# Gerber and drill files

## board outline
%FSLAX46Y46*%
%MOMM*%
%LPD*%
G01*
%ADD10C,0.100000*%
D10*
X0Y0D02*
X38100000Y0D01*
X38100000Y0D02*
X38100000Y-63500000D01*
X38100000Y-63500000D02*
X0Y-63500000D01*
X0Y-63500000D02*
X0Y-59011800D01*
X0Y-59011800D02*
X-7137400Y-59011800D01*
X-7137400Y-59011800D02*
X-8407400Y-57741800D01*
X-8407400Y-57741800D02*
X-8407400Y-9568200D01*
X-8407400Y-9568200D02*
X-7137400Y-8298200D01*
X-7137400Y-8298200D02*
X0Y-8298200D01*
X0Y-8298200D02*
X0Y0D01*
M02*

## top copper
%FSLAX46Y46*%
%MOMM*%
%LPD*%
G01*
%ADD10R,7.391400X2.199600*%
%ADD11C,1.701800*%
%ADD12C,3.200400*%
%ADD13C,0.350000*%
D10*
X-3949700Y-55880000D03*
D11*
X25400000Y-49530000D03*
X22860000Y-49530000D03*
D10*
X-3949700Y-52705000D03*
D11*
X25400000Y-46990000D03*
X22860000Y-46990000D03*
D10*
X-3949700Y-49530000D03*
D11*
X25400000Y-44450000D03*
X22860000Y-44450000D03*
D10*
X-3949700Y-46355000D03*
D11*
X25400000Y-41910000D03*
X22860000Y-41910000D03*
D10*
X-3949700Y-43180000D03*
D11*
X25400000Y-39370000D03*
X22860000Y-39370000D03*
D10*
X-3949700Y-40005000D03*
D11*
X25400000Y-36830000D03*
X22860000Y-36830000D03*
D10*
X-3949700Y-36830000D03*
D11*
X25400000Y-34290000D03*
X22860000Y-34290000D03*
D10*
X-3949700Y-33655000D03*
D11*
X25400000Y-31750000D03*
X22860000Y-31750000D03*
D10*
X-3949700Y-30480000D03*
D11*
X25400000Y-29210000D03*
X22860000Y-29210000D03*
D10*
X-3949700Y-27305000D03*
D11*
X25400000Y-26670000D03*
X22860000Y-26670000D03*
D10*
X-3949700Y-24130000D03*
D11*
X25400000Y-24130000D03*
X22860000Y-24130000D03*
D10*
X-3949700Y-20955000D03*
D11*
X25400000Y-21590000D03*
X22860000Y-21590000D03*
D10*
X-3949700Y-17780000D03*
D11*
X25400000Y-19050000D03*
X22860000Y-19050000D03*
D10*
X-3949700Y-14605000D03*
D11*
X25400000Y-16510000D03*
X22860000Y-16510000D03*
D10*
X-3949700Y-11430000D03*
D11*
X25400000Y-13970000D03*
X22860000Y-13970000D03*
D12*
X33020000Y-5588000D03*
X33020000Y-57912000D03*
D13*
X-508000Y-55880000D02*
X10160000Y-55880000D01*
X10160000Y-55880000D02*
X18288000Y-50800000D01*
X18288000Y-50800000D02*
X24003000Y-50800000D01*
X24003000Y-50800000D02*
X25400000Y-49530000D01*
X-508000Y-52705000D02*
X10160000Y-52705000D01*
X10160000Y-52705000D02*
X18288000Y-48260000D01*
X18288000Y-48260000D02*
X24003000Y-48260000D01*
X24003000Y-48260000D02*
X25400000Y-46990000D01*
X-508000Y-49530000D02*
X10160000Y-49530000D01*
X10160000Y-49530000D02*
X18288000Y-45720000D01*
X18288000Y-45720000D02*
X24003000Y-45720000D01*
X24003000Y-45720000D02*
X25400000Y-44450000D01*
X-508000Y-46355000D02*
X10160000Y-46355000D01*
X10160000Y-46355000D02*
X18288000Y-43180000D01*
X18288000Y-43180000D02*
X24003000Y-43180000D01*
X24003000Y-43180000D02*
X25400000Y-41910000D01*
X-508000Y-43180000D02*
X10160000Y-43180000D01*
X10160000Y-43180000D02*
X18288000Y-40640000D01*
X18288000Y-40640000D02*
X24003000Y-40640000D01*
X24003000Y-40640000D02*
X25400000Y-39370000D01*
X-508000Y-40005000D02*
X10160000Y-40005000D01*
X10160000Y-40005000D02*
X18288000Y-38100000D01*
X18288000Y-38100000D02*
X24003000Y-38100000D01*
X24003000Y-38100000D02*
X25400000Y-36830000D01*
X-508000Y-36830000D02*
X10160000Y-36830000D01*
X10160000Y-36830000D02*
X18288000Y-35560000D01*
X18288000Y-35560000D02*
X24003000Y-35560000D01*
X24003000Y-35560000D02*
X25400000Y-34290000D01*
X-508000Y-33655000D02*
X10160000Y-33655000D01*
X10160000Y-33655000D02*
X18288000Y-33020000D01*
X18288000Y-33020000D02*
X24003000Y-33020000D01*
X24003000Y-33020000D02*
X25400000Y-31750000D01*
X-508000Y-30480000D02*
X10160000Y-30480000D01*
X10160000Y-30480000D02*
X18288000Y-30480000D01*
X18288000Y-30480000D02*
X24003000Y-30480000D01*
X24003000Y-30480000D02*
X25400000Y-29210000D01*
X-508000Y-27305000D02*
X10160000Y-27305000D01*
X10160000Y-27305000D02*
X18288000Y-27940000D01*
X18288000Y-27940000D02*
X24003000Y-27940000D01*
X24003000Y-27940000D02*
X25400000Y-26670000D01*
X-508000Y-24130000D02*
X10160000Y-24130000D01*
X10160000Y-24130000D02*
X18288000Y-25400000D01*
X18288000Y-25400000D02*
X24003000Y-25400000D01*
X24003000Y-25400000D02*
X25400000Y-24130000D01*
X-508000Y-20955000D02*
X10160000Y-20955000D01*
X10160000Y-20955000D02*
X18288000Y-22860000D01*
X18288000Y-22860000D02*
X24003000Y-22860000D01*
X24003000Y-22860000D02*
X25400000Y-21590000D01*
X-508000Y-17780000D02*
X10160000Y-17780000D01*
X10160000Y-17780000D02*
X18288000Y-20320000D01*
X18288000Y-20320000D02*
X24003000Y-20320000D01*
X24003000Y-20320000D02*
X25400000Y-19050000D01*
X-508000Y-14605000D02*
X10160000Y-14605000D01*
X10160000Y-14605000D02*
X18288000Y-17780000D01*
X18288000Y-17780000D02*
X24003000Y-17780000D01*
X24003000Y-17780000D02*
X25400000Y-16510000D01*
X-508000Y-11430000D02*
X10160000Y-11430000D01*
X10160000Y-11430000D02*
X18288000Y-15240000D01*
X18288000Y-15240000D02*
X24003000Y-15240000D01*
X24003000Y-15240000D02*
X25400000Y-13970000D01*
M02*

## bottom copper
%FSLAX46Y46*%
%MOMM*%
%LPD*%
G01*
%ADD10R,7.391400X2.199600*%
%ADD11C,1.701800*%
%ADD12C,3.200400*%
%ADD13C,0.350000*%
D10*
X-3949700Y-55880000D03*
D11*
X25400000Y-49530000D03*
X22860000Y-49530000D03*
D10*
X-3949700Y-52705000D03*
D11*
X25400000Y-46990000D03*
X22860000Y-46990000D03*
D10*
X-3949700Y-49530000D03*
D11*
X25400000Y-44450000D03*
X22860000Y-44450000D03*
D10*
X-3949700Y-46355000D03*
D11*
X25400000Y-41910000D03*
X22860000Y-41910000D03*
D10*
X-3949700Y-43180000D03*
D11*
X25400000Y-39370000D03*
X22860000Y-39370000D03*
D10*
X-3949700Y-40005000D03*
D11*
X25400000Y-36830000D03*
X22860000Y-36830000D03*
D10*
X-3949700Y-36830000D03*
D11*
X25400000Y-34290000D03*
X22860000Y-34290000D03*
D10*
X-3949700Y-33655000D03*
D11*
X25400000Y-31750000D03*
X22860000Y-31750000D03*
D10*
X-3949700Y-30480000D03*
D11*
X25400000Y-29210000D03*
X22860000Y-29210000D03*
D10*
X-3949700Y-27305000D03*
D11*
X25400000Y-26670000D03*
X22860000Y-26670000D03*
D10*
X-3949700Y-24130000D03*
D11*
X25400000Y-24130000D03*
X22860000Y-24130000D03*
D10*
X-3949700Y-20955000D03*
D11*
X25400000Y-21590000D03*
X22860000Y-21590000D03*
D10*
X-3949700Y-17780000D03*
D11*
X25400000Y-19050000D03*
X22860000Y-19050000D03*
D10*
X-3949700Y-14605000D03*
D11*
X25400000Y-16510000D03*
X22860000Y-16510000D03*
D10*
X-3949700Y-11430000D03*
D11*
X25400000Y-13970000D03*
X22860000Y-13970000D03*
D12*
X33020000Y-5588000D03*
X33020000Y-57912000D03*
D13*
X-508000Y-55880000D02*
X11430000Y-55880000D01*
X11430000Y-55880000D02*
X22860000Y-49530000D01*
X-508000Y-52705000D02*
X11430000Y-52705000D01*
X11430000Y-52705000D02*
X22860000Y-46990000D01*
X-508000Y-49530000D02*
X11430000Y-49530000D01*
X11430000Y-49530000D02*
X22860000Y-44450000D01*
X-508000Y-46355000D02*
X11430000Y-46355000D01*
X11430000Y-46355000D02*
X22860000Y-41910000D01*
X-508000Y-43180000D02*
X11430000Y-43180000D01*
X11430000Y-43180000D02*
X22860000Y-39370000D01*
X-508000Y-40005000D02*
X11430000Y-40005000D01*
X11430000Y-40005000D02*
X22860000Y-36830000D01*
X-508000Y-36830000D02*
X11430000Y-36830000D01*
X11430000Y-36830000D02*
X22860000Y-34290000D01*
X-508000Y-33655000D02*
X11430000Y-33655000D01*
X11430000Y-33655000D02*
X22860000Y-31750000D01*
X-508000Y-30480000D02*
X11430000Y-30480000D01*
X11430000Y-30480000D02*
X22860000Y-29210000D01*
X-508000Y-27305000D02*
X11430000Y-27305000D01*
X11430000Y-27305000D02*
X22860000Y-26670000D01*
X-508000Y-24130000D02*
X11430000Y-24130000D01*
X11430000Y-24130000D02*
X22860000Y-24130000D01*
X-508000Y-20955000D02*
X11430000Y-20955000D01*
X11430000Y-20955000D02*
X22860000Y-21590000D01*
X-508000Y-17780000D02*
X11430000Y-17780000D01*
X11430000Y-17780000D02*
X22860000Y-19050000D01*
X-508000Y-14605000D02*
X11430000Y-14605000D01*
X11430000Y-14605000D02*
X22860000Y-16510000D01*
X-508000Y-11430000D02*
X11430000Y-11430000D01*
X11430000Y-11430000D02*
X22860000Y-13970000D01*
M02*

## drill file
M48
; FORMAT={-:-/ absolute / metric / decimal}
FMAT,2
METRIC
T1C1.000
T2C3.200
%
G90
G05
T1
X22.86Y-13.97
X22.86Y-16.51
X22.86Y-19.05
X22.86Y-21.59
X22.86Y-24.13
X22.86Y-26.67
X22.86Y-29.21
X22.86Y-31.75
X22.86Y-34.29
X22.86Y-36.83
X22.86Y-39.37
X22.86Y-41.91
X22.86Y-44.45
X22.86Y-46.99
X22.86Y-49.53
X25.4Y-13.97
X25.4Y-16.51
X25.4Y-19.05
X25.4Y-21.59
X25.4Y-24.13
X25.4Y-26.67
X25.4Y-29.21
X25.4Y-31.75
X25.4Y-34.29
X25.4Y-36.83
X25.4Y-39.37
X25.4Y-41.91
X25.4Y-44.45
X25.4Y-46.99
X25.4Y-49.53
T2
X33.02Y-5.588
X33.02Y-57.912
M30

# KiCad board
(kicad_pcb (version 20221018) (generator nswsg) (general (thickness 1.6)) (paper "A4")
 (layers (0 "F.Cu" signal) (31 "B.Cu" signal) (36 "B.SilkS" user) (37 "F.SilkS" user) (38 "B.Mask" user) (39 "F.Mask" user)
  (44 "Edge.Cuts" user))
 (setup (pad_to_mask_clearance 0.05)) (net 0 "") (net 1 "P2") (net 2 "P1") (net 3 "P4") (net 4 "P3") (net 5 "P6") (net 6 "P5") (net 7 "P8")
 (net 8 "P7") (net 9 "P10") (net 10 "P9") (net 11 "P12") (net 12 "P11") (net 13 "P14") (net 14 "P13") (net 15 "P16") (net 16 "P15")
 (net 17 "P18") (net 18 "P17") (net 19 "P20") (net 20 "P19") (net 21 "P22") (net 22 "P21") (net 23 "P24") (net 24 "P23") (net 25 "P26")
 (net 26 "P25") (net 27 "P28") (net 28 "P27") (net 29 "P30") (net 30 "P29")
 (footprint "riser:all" (layer "F.Cu") (at 0 0)
  (pad "2" smd rect (at -3.9497 55.88) (size 7.3914 2.1996) (layers "F.Cu" "F.Mask") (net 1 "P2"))
  (pad "1" smd rect (at -3.9497 55.88) (size 7.3914 2.1996) (layers "B.Cu" "B.Mask") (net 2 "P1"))
  (pad "2" thru_hole circle (at 25.4 49.53) (size 1.7018 1.7018) (drill 1.0) (layers "*.Cu" "*.Mask") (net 1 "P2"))
  (pad "1" thru_hole circle (at 22.86 49.53) (size 1.7018 1.7018) (drill 1.0) (layers "*.Cu" "*.Mask") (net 2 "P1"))
  (pad "4" smd rect (at -3.9497 52.705) (size 7.3914 2.1996) (layers "F.Cu" "F.Mask") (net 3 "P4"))
  (pad "3" smd rect (at -3.9497 52.705) (size 7.3914 2.1996) (layers "B.Cu" "B.Mask") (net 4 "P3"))
  (pad "4" thru_hole circle (at 25.4 46.99) (size 1.7018 1.7018) (drill 1.0) (layers "*.Cu" "*.Mask") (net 3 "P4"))
  (pad "3" thru_hole circle (at 22.86 46.99) (size 1.7018 1.7018) (drill 1.0) (layers "*.Cu" "*.Mask") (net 4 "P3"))
  (pad "6" smd rect (at -3.9497 49.53) (size 7.3914 2.1996) (layers "F.Cu" "F.Mask") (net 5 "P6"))
  (pad "5" smd rect (at -3.9497 49.53) (size 7.3914 2.1996) (layers "B.Cu" "B.Mask") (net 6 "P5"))
  (pad "6" thru_hole circle (at 25.4 44.45) (size 1.7018 1.7018) (drill 1.0) (layers "*.Cu" "*.Mask") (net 5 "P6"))
  (pad "5" thru_hole circle (at 22.86 44.45) (size 1.7018 1.7018) (drill 1.0) (layers "*.Cu" "*.Mask") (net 6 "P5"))
  (pad "8" smd rect (at -3.9497 46.355) (size 7.3914 2.1996) (layers "F.Cu" "F.Mask") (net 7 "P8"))
  (pad "7" smd rect (at -3.9497 46.355) (size 7.3914 2.1996) (layers "B.Cu" "B.Mask") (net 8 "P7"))
  (pad "8" thru_hole circle (at 25.4 41.91) (size 1.7018 1.7018) (drill 1.0) (layers "*.Cu" "*.Mask") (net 7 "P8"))
  (pad "7" thru_hole circle (at 22.86 41.91) (size 1.7018 1.7018) (drill 1.0) (layers "*.Cu" "*.Mask") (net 8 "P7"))
  (pad "10" smd rect (at -3.9497 43.18) (size 7.3914 2.1996) (layers "F.Cu" "F.Mask") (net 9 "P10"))
  (pad "9" smd rect (at -3.9497 43.18) (size 7.3914 2.1996) (layers "B.Cu" "B.Mask") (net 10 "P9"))
  (pad "10" thru_hole circle (at 25.4 39.37) (size 1.7018 1.7018) (drill 1.0) (layers "*.Cu" "*.Mask") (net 9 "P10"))
  (pad "9" thru_hole circle (at 22.86 39.37) (size 1.7018 1.7018) (drill 1.0) (layers "*.Cu" "*.Mask") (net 10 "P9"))
  (pad "12" smd rect (at -3.9497 40.005) (size 7.3914 2.1996) (layers "F.Cu" "F.Mask") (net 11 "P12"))
  (pad "11" smd rect (at -3.9497 40.005) (size 7.3914 2.1996) (layers "B.Cu" "B.Mask") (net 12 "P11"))
  (pad "12" thru_hole circle (at 25.4 36.83) (size 1.7018 1.7018) (drill 1.0) (layers "*.Cu" "*.Mask") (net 11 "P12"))
  (pad "11" thru_hole circle (at 22.86 36.83) (size 1.7018 1.7018) (drill 1.0) (layers "*.Cu" "*.Mask") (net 12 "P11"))
  (pad "14" smd rect (at -3.9497 36.83) (size 7.3914 2.1996) (layers "F.Cu" "F.Mask") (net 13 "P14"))
  (pad "13" smd rect (at -3.9497 36.83) (size 7.3914 2.1996) (layers "B.Cu" "B.Mask") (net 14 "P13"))
  (pad "14" thru_hole circle (at 25.4 34.29) (size 1.7018 1.7018) (drill 1.0) (layers "*.Cu" "*.Mask") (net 13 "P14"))
  (pad "13" thru_hole circle (at 22.86 34.29) (size 1.7018 1.7018) (drill 1.0) (layers "*.Cu" "*.Mask") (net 14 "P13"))
  (pad "16" smd rect (at -3.9497 33.655) (size 7.3914 2.1996) (layers "F.Cu" "F.Mask") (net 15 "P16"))
  (pad "15" smd rect (at -3.9497 33.655) (size 7.3914 2.1996) (layers "B.Cu" "B.Mask") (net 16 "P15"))
  (pad "16" thru_hole circle (at 25.4 31.75) (size 1.7018 1.7018) (drill 1.0) (layers "*.Cu" "*.Mask") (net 15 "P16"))
  (pad "15" thru_hole circle (at 22.86 31.75) (size 1.7018 1.7018) (drill 1.0) (layers "*.Cu" "*.Mask") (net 16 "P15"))
  (pad "18" smd rect (at -3.9497 30.48) (size 7.3914 2.1996) (layers "F.Cu" "F.Mask") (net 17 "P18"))
  (pad "17" smd rect (at -3.9497 30.48) (size 7.3914 2.1996) (layers "B.Cu" "B.Mask") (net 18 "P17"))
  (pad "18" thru_hole circle (at 25.4 29.21) (size 1.7018 1.7018) (drill 1.0) (layers "*.Cu" "*.Mask") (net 17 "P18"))
  (pad "17" thru_hole circle (at 22.86 29.21) (size 1.7018 1.7018) (drill 1.0) (layers "*.Cu" "*.Mask") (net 18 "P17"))
  (pad "20" smd rect (at -3.9497 27.305) (size 7.3914 2.1996) (layers "F.Cu" "F.Mask") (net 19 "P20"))
  (pad "19" smd rect (at -3.9497 27.305) (size 7.3914 2.1996) (layers "B.Cu" "B.Mask") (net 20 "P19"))
  (pad "20" thru_hole circle (at 25.4 26.67) (size 1.7018 1.7018) (drill 1.0) (layers "*.Cu" "*.Mask") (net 19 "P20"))
  (pad "19" thru_hole circle (at 22.86 26.67) (size 1.7018 1.7018) (drill 1.0) (layers "*.Cu" "*.Mask") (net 20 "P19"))
  (pad "22" smd rect (at -3.9497 24.13) (size 7.3914 2.1996) (layers "F.Cu" "F.Mask") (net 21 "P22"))
  (pad "21" smd rect (at -3.9497 24.13) (size 7.3914 2.1996) (layers "B.Cu" "B.Mask") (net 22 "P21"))
  (pad "22" thru_hole circle (at 25.4 24.13) (size 1.7018 1.7018) (drill 1.0) (layers "*.Cu" "*.Mask") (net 21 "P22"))
  (pad "21" thru_hole circle (at 22.86 24.13) (size 1.7018 1.7018) (drill 1.0) (layers "*.Cu" "*.Mask") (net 22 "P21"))
  (pad "24" smd rect (at -3.9497 20.955) (size 7.3914 2.1996) (layers "F.Cu" "F.Mask") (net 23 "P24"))
  (pad "23" smd rect (at -3.9497 20.955) (size 7.3914 2.1996) (layers "B.Cu" "B.Mask") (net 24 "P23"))
  (pad "24" thru_hole circle (at 25.4 21.59) (size 1.7018 1.7018) (drill 1.0) (layers "*.Cu" "*.Mask") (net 23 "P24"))
  (pad "23" thru_hole circle (at 22.86 21.59) (size 1.7018 1.7018) (drill 1.0) (layers "*.Cu" "*.Mask") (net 24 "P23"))
  (pad "26" smd rect (at -3.9497 17.78) (size 7.3914 2.1996) (layers "F.Cu" "F.Mask") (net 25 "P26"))
  (pad "25" smd rect (at -3.9497 17.78) (size 7.3914 2.1996) (layers "B.Cu" "B.Mask") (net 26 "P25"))
  (pad "26" thru_hole circle (at 25.4 19.05) (size 1.7018 1.7018) (drill 1.0) (layers "*.Cu" "*.Mask") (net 25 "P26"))
  (pad "25" thru_hole circle (at 22.86 19.05) (size 1.7018 1.7018) (drill 1.0) (layers "*.Cu" "*.Mask") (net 26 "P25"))
  (pad "28" smd rect (at -3.9497 14.605) (size 7.3914 2.1996) (layers "F.Cu" "F.Mask") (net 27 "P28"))
  (pad "27" smd rect (at -3.9497 14.605) (size 7.3914 2.1996) (layers "B.Cu" "B.Mask") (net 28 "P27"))
  (pad "28" thru_hole circle (at 25.4 16.51) (size 1.7018 1.7018) (drill 1.0) (layers "*.Cu" "*.Mask") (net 27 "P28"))
  (pad "27" thru_hole circle (at 22.86 16.51) (size 1.7018 1.7018) (drill 1.0) (layers "*.Cu" "*.Mask") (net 28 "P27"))
  (pad "30" smd rect (at -3.9497 11.43) (size 7.3914 2.1996) (layers "F.Cu" "F.Mask") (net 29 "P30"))
  (pad "29" smd rect (at -3.9497 11.43) (size 7.3914 2.1996) (layers "B.Cu" "B.Mask") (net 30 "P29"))
  (pad "30" thru_hole circle (at 25.4 13.97) (size 1.7018 1.7018) (drill 1.0) (layers "*.Cu" "*.Mask") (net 29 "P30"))
  (pad "29" thru_hole circle (at 22.86 13.97) (size 1.7018 1.7018) (drill 1.0) (layers "*.Cu" "*.Mask") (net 30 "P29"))
  (pad "" np_thru_hole circle (at 33.02 5.588) (size 3.2004 3.2004) (drill 3.2) (layers "*.Cu" "*.Mask"))
  (pad "" np_thru_hole circle (at 33.02 57.912) (size 3.2004 3.2004) (drill 3.2) (layers "*.Cu" "*.Mask")))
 (gr_line (start 0.0 0.0) (end 38.1 0.0) (layer "Edge.Cuts") (width 0.1))
 (gr_line (start 38.1 0.0) (end 38.1 63.5) (layer "Edge.Cuts") (width 0.1))
 (gr_line (start 38.1 63.5) (end 0.0 63.5) (layer "Edge.Cuts") (width 0.1))
 (gr_line (start 0.0 63.5) (end 0.0 59.0118) (layer "Edge.Cuts") (width 0.1))
 (gr_line (start 0.0 59.0118) (end -7.1374 59.0118) (layer "Edge.Cuts") (width 0.1))
 (gr_line (start -7.1374 59.0118) (end -8.4074 57.7418) (layer "Edge.Cuts") (width 0.1))
 (gr_line (start -8.4074 57.7418) (end -8.4074 9.5682) (layer "Edge.Cuts") (width 0.1))
 (gr_line (start -8.4074 9.5682) (end -7.1374 8.2982) (layer "Edge.Cuts") (width 0.1))
 (gr_line (start -7.1374 8.2982) (end 0.0 8.2982) (layer "Edge.Cuts") (width 0.1))
 (gr_line (start 0.0 8.2982) (end 0.0 0.0) (layer "Edge.Cuts") (width 0.1))
 (segment (start -0.508 55.88) (end 10.16 55.88) (width 0.35) (layer "F.Cu") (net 1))
 (segment (start 10.16 55.88) (end 18.288 50.8) (width 0.35) (layer "F.Cu") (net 1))
 (segment (start 18.288 50.8) (end 24.003 50.8) (width 0.35) (layer "F.Cu") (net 1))
 (segment (start 24.003 50.8) (end 25.4 49.53) (width 0.35) (layer "F.Cu") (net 1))
 (segment (start -0.508 55.88) (end 11.43 55.88) (width 0.35) (layer "B.Cu") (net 2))
 (segment (start 11.43 55.88) (end 22.86 49.53) (width 0.35) (layer "B.Cu") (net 2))
 (segment (start -0.508 52.705) (end 10.16 52.705) (width 0.35) (layer "F.Cu") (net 3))
 (segment (start 10.16 52.705) (end 18.288 48.26) (width 0.35) (layer "F.Cu") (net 3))
 (segment (start 18.288 48.26) (end 24.003 48.26) (width 0.35) (layer "F.Cu") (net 3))
 (segment (start 24.003 48.26) (end 25.4 46.99) (width 0.35) (layer "F.Cu") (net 3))
 (segment (start -0.508 52.705) (end 11.43 52.705) (width 0.35) (layer "B.Cu") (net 4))
 (segment (start 11.43 52.705) (end 22.86 46.99) (width 0.35) (layer "B.Cu") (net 4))
 (segment (start -0.508 49.53) (end 10.16 49.53) (width 0.35) (layer "F.Cu") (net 5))
 (segment (start 10.16 49.53) (end 18.288 45.72) (width 0.35) (layer "F.Cu") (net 5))
 (segment (start 18.288 45.72) (end 24.003 45.72) (width 0.35) (layer "F.Cu") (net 5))
 (segment (start 24.003 45.72) (end 25.4 44.45) (width 0.35) (layer "F.Cu") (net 5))
 (segment (start -0.508 49.53) (end 11.43 49.53) (width 0.35) (layer "B.Cu") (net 6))
 (segment (start 11.43 49.53) (end 22.86 44.45) (width 0.35) (layer "B.Cu") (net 6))
 (segment (start -0.508 46.355) (end 10.16 46.355) (width 0.35) (layer "F.Cu") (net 7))
 (segment (start 10.16 46.355) (end 18.288 43.18) (width 0.35) (layer "F.Cu") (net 7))
 (segment (start 18.288 43.18) (end 24.003 43.18) (width 0.35) (layer "F.Cu") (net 7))
 (segment (start 24.003 43.18) (end 25.4 41.91) (width 0.35) (layer "F.Cu") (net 7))
 (segment (start -0.508 46.355) (end 11.43 46.355) (width 0.35) (layer "B.Cu") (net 8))
 (segment (start 11.43 46.355) (end 22.86 41.91) (width 0.35) (layer "B.Cu") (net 8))
 (segment (start -0.508 43.18) (end 10.16 43.18) (width 0.35) (layer "F.Cu") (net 9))
 (segment (start 10.16 43.18) (end 18.288 40.64) (width 0.35) (layer "F.Cu") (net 9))
 (segment (start 18.288 40.64) (end 24.003 40.64) (width 0.35) (layer "F.Cu") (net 9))
 (segment (start 24.003 40.64) (end 25.4 39.37) (width 0.35) (layer "F.Cu") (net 9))
 (segment (start -0.508 43.18) (end 11.43 43.18) (width 0.35) (layer "B.Cu") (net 10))
 (segment (start 11.43 43.18) (end 22.86 39.37) (width 0.35) (layer "B.Cu") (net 10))
 (segment (start -0.508 40.005) (end 10.16 40.005) (width 0.35) (layer "F.Cu") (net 11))
 (segment (start 10.16 40.005) (end 18.288 38.1) (width 0.35) (layer "F.Cu") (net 11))
 (segment (start 18.288 38.1) (end 24.003 38.1) (width 0.35) (layer "F.Cu") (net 11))
 (segment (start 24.003 38.1) (end 25.4 36.83) (width 0.35) (layer "F.Cu") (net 11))
 (segment (start -0.508 40.005) (end 11.43 40.005) (width 0.35) (layer "B.Cu") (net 12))
 (segment (start 11.43 40.005) (end 22.86 36.83) (width 0.35) (layer "B.Cu") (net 12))
 (segment (start -0.508 36.83) (end 10.16 36.83) (width 0.35) (layer "F.Cu") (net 13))
 (segment (start 10.16 36.83) (end 18.288 35.56) (width 0.35) (layer "F.Cu") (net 13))
 (segment (start 18.288 35.56) (end 24.003 35.56) (width 0.35) (layer "F.Cu") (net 13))
 (segment (start 24.003 35.56) (end 25.4 34.29) (width 0.35) (layer "F.Cu") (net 13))
 (segment (start -0.508 36.83) (end 11.43 36.83) (width 0.35) (layer "B.Cu") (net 14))
 (segment (start 11.43 36.83) (end 22.86 34.29) (width 0.35) (layer "B.Cu") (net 14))
 (segment (start -0.508 33.655) (end 10.16 33.655) (width 0.35) (layer "F.Cu") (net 15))
 (segment (start 10.16 33.655) (end 18.288 33.02) (width 0.35) (layer "F.Cu") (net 15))
 (segment (start 18.288 33.02) (end 24.003 33.02) (width 0.35) (layer "F.Cu") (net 15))
 (segment (start 24.003 33.02) (end 25.4 31.75) (width 0.35) (layer "F.Cu") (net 15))
 (segment (start -0.508 33.655) (end 11.43 33.655) (width 0.35) (layer "B.Cu") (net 16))
 (segment (start 11.43 33.655) (end 22.86 31.75) (width 0.35) (layer "B.Cu") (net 16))
 (segment (start -0.508 30.48) (end 10.16 30.48) (width 0.35) (layer "F.Cu") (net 17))
 (segment (start 10.16 30.48) (end 18.288 30.48) (width 0.35) (layer "F.Cu") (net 17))
 (segment (start 18.288 30.48) (end 24.003 30.48) (width 0.35) (layer "F.Cu") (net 17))
 (segment (start 24.003 30.48) (end 25.4 29.21) (width 0.35) (layer "F.Cu") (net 17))
 (segment (start -0.508 30.48) (end 11.43 30.48) (width 0.35) (layer "B.Cu") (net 18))
 (segment (start 11.43 30.48) (end 22.86 29.21) (width 0.35) (layer "B.Cu") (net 18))
 (segment (start -0.508 27.305) (end 10.16 27.305) (width 0.35) (layer "F.Cu") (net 19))
 (segment (start 10.16 27.305) (end 18.288 27.94) (width 0.35) (layer "F.Cu") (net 19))
 (segment (start 18.288 27.94) (end 24.003 27.94) (width 0.35) (layer "F.Cu") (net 19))
 (segment (start 24.003 27.94) (end 25.4 26.67) (width 0.35) (layer "F.Cu") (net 19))
 (segment (start -0.508 27.305) (end 11.43 27.305) (width 0.35) (layer "B.Cu") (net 20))
 (segment (start 11.43 27.305) (end 22.86 26.67) (width 0.35) (layer "B.Cu") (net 20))
 (segment (start -0.508 24.13) (end 10.16 24.13) (width 0.35) (layer "F.Cu") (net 21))
 (segment (start 10.16 24.13) (end 18.288 25.4) (width 0.35) (layer "F.Cu") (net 21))
 (segment (start 18.288 25.4) (end 24.003 25.4) (width 0.35) (layer "F.Cu") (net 21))
 (segment (start 24.003 25.4) (end 25.4 24.13) (width 0.35) (layer "F.Cu") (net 21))
 (segment (start -0.508 24.13) (end 11.43 24.13) (width 0.35) (layer "B.Cu") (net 22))
 (segment (start 11.43 24.13) (end 22.86 24.13) (width 0.35) (layer "B.Cu") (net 22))
 (segment (start -0.508 20.955) (end 10.16 20.955) (width 0.35) (layer "F.Cu") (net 23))
 (segment (start 10.16 20.955) (end 18.288 22.86) (width 0.35) (layer "F.Cu") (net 23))
 (segment (start 18.288 22.86) (end 24.003 22.86) (width 0.35) (layer "F.Cu") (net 23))
 (segment (start 24.003 22.86) (end 25.4 21.59) (width 0.35) (layer "F.Cu") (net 23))
 (segment (start -0.508 20.955) (end 11.43 20.955) (width 0.35) (layer "B.Cu") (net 24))
 (segment (start 11.43 20.955) (end 22.86 21.59) (width 0.35) (layer "B.Cu") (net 24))
 (segment (start -0.508 17.78) (end 10.16 17.78) (width 0.35) (layer "F.Cu") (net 25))
 (segment (start 10.16 17.78) (end 18.288 20.32) (width 0.35) (layer "F.Cu") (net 25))
 (segment (start 18.288 20.32) (end 24.003 20.32) (width 0.35) (layer "F.Cu") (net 25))
 (segment (start 24.003 20.32) (end 25.4 19.05) (width 0.35) (layer "F.Cu") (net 25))
 (segment (start -0.508 17.78) (end 11.43 17.78) (width 0.35) (layer "B.Cu") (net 26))
 (segment (start 11.43 17.78) (end 22.86 19.05) (width 0.35) (layer "B.Cu") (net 26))
 (segment (start -0.508 14.605) (end 10.16 14.605) (width 0.35) (layer "F.Cu") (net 27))
 (segment (start 10.16 14.605) (end 18.288 17.78) (width 0.35) (layer "F.Cu") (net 27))
 (segment (start 18.288 17.78) (end 24.003 17.78) (width 0.35) (layer "F.Cu") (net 27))
 (segment (start 24.003 17.78) (end 25.4 16.51) (width 0.35) (layer "F.Cu") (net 27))
 (segment (start -0.508 14.605) (end 11.43 14.605) (width 0.35) (layer "B.Cu") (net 28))
 (segment (start 11.43 14.605) (end 22.86 16.51) (width 0.35) (layer "B.Cu") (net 28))
 (segment (start -0.508 11.43) (end 10.16 11.43) (width 0.35) (layer "F.Cu") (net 29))
 (segment (start 10.16 11.43) (end 18.288 15.24) (width 0.35) (layer "F.Cu") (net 29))
 (segment (start 18.288 15.24) (end 24.003 15.24) (width 0.35) (layer "F.Cu") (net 29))
 (segment (start 24.003 15.24) (end 25.4 13.97) (width 0.35) (layer "F.Cu") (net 29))
 (segment (start -0.508 11.43) (end 11.43 11.43) (width 0.35) (layer "B.Cu") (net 30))
 (segment (start 11.43 11.43) (end 22.86 13.97) (width 0.35) (layer "B.Cu") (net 30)))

